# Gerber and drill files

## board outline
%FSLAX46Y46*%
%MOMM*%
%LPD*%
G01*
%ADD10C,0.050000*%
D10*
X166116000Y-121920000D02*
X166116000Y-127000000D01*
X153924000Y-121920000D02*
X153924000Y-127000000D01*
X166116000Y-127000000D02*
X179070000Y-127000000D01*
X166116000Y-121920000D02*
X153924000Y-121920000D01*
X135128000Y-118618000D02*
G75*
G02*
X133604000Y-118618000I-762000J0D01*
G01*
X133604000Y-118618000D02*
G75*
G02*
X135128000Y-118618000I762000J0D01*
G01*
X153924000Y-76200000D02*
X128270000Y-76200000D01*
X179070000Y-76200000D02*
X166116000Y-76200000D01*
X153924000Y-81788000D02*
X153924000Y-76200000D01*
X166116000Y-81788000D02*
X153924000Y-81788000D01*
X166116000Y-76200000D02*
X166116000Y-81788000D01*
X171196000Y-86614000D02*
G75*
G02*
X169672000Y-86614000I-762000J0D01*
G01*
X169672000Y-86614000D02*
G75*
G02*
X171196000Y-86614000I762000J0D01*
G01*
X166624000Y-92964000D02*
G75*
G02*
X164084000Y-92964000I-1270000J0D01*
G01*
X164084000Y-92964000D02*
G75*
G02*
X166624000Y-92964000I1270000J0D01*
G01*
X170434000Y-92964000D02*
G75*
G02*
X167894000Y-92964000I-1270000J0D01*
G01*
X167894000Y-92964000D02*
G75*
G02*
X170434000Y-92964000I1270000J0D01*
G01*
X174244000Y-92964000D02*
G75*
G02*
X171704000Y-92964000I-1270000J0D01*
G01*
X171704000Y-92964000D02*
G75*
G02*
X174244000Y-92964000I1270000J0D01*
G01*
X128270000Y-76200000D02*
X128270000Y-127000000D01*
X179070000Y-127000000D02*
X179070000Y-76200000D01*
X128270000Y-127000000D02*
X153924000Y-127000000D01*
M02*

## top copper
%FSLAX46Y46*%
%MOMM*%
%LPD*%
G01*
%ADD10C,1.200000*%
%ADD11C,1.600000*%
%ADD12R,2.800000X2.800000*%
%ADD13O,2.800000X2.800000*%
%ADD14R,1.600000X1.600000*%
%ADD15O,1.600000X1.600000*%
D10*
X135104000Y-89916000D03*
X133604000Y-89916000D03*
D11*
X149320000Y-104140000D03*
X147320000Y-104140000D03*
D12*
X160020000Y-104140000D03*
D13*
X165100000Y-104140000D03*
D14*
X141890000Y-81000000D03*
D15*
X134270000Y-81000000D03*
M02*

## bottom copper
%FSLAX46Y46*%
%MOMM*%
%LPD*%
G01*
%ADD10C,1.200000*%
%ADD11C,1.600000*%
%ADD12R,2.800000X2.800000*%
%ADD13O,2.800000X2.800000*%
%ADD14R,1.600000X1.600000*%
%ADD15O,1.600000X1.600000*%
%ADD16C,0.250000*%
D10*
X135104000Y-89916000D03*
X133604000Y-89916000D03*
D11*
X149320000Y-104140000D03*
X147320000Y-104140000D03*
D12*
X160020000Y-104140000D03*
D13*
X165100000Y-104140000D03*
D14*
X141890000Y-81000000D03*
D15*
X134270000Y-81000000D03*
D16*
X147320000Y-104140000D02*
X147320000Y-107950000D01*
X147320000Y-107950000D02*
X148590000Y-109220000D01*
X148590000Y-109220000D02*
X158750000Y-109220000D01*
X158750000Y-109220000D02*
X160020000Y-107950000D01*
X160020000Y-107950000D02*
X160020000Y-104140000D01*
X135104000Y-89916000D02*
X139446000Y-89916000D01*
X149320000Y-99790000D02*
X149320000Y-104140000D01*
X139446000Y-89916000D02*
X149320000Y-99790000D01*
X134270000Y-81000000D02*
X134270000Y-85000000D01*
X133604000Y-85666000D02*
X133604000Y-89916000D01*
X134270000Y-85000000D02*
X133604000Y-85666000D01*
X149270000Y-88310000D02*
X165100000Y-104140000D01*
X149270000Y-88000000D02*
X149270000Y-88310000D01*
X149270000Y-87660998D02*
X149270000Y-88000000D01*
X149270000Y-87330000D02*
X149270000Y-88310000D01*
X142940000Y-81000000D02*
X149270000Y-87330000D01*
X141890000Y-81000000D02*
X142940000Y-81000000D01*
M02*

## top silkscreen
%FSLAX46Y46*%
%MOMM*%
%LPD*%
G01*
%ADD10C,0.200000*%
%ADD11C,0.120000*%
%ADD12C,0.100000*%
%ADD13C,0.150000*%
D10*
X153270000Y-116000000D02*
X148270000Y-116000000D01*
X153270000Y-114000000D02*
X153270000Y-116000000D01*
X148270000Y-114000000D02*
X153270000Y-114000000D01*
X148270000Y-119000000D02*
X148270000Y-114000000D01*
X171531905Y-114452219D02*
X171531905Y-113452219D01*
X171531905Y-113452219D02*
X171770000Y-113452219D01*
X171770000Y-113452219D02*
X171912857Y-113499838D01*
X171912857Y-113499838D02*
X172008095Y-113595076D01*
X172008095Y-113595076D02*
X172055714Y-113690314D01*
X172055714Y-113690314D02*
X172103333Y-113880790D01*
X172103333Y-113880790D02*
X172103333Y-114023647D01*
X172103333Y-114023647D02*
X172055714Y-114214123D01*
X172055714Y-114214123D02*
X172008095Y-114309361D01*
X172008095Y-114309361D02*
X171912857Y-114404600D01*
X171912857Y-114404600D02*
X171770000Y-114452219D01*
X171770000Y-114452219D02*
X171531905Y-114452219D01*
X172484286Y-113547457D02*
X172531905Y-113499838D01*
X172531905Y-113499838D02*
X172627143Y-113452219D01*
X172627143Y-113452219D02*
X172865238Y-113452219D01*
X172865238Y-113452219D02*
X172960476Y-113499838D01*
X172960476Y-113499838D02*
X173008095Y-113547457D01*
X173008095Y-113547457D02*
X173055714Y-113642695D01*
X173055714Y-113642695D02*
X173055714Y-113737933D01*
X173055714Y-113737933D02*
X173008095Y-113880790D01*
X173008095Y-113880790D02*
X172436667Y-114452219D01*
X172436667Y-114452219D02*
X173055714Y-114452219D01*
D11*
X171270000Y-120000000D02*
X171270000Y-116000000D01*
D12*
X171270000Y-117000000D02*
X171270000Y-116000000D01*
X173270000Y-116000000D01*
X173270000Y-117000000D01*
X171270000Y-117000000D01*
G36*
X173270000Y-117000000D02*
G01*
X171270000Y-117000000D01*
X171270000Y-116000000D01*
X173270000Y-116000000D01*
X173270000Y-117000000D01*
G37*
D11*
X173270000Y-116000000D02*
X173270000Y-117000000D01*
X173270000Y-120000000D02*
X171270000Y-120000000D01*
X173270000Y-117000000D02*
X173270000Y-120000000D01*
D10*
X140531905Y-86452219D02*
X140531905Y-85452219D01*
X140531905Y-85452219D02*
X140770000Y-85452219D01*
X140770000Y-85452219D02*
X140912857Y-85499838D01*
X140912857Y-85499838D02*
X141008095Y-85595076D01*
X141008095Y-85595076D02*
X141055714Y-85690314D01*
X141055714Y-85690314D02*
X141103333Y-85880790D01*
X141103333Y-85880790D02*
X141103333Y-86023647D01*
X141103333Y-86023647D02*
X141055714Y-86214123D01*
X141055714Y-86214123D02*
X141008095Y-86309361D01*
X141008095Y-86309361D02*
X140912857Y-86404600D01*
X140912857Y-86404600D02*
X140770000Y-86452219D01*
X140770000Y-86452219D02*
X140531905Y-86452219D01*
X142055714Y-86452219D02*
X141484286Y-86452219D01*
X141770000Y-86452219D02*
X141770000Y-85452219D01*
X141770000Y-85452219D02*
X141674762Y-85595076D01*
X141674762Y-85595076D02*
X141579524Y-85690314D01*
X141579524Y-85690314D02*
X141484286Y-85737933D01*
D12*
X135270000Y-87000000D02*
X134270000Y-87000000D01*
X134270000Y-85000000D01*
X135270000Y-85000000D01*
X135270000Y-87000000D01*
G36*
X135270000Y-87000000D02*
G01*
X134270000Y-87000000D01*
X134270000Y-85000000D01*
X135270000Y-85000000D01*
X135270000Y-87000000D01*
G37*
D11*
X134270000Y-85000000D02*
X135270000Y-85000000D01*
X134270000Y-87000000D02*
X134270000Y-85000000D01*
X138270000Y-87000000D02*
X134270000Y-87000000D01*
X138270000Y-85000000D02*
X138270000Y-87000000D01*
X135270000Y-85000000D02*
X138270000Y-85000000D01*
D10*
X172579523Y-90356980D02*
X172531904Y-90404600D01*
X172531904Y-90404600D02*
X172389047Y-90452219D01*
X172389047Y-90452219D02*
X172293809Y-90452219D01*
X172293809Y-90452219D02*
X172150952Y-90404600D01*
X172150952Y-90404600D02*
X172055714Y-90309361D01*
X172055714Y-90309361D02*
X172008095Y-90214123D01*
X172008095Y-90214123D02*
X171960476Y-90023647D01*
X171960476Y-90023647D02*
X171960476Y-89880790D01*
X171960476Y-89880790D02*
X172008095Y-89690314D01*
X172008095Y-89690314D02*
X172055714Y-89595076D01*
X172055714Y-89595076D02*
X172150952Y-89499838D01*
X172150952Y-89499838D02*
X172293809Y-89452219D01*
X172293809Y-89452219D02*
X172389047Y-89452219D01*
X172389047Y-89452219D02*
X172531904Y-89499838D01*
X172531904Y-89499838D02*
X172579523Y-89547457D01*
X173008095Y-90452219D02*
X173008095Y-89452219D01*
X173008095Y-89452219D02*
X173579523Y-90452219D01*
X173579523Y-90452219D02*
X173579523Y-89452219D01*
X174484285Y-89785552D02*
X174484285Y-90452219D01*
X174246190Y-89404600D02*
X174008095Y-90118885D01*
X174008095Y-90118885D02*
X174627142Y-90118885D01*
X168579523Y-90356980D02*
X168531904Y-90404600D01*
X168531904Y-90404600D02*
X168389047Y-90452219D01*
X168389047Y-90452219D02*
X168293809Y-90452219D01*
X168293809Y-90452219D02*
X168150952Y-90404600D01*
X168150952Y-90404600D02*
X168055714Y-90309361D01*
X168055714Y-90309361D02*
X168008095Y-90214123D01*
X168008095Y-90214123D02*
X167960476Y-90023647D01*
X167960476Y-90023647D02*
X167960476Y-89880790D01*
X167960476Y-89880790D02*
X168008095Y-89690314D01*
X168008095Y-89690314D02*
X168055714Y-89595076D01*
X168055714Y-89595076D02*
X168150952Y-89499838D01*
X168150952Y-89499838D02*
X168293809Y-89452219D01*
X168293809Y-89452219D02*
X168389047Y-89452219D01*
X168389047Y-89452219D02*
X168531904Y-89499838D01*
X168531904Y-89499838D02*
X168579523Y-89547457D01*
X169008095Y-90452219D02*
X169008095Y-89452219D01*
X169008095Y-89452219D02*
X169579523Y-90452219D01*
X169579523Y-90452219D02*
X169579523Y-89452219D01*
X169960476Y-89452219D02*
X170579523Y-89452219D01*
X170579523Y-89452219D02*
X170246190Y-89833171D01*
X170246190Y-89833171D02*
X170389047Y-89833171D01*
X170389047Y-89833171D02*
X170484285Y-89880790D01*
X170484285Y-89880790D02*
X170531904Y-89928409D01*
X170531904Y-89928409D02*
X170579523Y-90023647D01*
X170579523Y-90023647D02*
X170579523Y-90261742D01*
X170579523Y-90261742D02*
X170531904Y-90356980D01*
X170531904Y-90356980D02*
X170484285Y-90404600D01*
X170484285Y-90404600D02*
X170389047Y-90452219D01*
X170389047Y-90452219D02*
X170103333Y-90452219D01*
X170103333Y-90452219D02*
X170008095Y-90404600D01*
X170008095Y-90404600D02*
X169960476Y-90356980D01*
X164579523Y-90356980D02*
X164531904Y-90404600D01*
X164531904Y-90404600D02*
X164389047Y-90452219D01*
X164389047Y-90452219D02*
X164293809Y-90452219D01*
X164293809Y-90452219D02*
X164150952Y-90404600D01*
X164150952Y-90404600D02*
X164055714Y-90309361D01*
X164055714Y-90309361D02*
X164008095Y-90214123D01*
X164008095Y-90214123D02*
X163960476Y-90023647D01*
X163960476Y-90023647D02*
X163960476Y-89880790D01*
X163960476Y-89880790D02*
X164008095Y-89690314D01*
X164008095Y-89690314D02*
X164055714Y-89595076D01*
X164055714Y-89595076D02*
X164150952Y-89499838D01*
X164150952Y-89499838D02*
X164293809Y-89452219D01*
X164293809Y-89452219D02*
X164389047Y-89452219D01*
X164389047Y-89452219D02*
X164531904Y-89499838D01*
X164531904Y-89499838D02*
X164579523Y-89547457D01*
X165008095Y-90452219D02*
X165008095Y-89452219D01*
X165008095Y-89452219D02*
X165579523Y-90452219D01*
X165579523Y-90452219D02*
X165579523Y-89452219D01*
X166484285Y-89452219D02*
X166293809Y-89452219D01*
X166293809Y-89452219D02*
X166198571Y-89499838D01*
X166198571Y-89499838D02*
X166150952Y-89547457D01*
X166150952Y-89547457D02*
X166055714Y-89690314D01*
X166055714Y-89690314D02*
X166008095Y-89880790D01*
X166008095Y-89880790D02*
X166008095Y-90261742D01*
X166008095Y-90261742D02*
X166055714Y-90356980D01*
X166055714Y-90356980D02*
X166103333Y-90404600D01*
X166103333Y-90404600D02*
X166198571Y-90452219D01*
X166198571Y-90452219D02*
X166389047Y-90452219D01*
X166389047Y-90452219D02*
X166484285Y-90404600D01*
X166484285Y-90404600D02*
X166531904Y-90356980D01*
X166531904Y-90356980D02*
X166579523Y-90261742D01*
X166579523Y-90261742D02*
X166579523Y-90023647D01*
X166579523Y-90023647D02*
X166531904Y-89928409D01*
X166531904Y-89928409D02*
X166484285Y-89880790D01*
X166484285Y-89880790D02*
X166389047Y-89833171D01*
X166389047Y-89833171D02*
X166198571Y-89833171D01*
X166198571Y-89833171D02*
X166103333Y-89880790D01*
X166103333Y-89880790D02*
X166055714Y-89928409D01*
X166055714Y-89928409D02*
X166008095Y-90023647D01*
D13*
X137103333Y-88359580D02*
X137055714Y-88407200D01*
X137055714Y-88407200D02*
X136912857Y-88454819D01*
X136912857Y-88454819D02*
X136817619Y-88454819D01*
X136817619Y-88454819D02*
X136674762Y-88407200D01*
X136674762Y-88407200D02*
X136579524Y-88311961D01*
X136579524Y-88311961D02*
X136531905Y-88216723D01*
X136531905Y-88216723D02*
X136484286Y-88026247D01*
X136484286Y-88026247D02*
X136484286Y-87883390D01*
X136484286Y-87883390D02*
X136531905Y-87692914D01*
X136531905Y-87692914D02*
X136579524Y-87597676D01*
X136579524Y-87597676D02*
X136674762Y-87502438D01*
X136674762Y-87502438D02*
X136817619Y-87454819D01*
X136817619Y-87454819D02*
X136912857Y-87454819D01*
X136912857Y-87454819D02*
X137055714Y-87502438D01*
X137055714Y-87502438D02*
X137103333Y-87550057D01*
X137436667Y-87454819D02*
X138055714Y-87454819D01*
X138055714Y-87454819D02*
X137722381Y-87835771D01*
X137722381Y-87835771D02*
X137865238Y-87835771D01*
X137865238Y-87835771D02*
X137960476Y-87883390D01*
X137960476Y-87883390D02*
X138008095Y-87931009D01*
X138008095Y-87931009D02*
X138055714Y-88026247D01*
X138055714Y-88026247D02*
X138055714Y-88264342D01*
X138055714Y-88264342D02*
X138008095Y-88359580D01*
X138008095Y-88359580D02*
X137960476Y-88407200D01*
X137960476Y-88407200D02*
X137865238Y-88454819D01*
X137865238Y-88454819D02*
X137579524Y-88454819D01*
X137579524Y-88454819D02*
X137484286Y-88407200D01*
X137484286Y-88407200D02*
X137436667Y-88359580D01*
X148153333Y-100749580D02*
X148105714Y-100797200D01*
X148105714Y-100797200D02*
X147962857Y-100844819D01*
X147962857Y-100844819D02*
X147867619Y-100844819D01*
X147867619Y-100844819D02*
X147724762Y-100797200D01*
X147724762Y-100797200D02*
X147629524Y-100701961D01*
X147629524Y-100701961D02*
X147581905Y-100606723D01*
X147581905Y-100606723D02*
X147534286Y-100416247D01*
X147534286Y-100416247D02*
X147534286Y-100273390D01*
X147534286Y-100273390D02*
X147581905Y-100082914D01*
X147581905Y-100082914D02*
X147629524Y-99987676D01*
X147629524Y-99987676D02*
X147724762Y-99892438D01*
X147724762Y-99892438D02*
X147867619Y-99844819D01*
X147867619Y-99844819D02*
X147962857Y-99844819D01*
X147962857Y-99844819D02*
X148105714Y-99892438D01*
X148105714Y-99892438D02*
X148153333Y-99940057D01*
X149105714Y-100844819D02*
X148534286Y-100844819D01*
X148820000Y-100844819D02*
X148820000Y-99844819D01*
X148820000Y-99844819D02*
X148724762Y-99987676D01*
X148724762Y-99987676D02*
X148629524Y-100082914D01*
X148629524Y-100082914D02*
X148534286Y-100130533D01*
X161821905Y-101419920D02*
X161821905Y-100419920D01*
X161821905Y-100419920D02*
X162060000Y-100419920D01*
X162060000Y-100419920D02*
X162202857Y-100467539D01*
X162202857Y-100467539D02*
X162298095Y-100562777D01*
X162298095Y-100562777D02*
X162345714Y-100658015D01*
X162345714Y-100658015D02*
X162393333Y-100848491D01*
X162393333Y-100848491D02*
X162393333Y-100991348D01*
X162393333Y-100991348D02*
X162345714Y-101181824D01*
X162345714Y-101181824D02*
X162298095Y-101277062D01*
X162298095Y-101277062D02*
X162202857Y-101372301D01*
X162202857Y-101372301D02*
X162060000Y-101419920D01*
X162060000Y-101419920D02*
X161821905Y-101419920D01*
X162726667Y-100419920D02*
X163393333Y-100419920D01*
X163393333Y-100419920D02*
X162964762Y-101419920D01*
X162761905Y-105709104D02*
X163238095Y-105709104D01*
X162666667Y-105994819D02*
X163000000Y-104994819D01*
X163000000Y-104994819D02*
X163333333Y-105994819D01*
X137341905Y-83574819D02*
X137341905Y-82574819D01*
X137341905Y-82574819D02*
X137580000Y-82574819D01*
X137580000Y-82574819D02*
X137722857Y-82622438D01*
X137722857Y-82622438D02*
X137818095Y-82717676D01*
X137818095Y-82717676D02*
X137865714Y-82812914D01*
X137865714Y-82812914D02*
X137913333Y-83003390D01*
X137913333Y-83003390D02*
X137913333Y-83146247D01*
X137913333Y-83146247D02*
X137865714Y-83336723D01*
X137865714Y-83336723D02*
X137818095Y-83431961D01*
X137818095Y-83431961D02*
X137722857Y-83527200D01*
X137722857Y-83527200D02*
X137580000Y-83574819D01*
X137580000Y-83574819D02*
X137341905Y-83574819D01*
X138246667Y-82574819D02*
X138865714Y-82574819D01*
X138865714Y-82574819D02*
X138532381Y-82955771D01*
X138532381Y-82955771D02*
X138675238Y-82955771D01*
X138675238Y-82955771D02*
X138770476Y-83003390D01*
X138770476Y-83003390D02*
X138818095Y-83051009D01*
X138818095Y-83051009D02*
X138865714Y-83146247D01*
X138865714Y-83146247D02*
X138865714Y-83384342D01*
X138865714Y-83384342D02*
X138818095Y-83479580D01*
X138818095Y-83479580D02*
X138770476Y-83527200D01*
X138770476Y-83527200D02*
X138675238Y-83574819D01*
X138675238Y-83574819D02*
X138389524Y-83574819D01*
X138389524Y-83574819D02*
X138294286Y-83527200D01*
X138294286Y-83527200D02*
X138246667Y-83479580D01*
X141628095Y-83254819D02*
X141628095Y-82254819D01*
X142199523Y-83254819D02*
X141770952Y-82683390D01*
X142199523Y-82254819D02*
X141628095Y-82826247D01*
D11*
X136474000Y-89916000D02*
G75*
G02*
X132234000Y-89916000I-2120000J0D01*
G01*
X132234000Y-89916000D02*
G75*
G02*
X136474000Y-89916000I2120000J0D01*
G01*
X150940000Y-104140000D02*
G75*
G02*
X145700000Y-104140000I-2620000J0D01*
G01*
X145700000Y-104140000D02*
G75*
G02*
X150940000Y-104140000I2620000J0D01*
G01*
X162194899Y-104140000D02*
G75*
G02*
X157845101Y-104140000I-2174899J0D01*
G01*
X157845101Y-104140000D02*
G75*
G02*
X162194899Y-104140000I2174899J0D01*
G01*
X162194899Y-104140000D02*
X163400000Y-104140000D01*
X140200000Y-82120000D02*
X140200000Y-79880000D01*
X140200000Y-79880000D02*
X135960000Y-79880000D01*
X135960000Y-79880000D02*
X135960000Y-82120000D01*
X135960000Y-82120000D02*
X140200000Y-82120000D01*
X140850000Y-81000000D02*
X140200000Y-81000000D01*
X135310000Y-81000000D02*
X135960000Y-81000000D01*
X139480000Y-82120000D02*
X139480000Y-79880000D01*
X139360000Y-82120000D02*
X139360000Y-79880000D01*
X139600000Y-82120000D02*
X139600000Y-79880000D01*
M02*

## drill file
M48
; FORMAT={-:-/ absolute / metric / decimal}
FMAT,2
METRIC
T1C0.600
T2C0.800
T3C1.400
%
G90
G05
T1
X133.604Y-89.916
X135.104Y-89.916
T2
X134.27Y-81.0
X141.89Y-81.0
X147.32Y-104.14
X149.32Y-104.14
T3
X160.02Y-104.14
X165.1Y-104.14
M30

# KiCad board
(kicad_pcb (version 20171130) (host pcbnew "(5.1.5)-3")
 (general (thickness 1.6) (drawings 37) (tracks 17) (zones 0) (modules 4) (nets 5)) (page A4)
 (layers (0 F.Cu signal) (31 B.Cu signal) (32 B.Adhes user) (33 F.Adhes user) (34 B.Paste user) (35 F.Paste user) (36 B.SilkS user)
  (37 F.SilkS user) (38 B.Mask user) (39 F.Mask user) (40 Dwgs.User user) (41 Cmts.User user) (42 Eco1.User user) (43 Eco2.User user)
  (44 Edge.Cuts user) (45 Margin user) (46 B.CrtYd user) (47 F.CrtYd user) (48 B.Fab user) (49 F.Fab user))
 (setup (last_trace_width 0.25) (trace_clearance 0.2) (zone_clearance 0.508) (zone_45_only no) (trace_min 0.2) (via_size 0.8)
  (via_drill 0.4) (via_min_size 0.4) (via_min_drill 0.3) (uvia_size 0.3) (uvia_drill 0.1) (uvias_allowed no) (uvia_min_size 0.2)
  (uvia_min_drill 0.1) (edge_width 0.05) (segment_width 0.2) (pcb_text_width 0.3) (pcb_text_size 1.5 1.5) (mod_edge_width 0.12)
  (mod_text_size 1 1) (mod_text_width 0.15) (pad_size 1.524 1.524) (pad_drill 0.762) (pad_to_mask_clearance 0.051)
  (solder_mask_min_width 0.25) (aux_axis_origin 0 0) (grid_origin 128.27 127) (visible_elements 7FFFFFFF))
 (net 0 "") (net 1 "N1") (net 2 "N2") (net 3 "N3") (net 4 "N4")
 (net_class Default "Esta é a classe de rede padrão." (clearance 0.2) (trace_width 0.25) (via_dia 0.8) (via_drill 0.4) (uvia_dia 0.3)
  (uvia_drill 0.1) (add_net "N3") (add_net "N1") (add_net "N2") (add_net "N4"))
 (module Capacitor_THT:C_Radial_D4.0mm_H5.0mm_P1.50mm (layer F.Cu) (at 133.604 89.916)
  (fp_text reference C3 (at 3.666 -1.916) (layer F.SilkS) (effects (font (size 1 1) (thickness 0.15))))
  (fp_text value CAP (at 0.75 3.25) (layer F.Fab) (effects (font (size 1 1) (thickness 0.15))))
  (fp_circle (center 0.75 0) (end 2.87 0) (layer F.SilkS) (width 0.12))
  (pad 2 thru_hole circle (at 1.5 0) (size 1.2 1.2) (drill 0.6) (layers *.Cu *.Mask) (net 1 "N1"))
  (pad 1 thru_hole circle (at 0 0) (size 1.2 1.2) (drill 0.6) (layers *.Cu *.Mask) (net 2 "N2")))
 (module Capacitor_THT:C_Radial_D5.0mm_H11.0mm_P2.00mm (layer F.Cu) (at 147.32 104.14)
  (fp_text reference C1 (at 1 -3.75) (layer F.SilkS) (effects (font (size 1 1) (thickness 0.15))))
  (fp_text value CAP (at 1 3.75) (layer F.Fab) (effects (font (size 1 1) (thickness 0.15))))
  (fp_circle (center 1 0) (end 3.62 0) (layer F.SilkS) (width 0.12))
  (pad 2 thru_hole circle (at 2 0) (size 1.6 1.6) (drill 0.8) (layers *.Cu *.Mask) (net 1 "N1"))
  (pad 1 thru_hole circle (at 0 0) (size 1.6 1.6) (drill 0.8) (layers *.Cu *.Mask) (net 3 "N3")))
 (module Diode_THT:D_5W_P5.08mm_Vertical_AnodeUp (layer F.Cu) (at 160.02 104.14)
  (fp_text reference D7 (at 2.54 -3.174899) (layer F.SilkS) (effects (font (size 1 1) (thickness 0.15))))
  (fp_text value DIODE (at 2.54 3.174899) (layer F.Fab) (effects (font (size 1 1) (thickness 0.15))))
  (fp_circle (center 0 0) (end 2.174899 0) (layer F.SilkS) (width 0.12))
  (fp_line (start 2.174899 0) (end 3.38 0) (layer F.SilkS) (width 0.12))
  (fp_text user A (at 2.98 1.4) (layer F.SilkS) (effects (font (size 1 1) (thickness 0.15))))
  (pad 1 thru_hole rect (at 0 0) (size 2.8 2.8) (drill 1.4) (layers *.Cu *.Mask) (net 3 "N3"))
  (pad 2 thru_hole oval (at 5.08 0) (size 2.8 2.8) (drill 1.4) (layers *.Cu *.Mask) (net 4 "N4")))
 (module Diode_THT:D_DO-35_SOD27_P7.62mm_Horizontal (layer F.Cu) (at 141.89 81 180)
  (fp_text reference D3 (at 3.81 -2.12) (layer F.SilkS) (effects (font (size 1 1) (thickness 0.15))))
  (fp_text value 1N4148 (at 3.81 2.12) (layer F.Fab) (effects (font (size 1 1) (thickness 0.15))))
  (fp_line (start 1.69 -1.12) (end 1.69 1.12) (layer F.SilkS) (width 0.12))
  (fp_line (start 1.69 1.12) (end 5.93 1.12) (layer F.SilkS) (width 0.12))
  (fp_line (start 5.93 1.12) (end 5.93 -1.12) (layer F.SilkS) (width 0.12))
  (fp_line (start 5.93 -1.12) (end 1.69 -1.12) (layer F.SilkS) (width 0.12))
  (fp_line (start 1.04 0) (end 1.69 0) (layer F.SilkS) (width 0.12))
  (fp_line (start 6.58 0) (end 5.93 0) (layer F.SilkS) (width 0.12))
  (fp_line (start 2.41 -1.12) (end 2.41 1.12) (layer F.SilkS) (width 0.12))
  (fp_line (start 2.53 -1.12) (end 2.53 1.12) (layer F.SilkS) (width 0.12))
  (fp_line (start 2.29 -1.12) (end 2.29 1.12) (layer F.SilkS) (width 0.12))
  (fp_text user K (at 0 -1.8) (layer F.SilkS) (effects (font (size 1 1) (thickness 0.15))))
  (pad 1 thru_hole rect (at 0 0 180) (size 1.6 1.6) (drill 0.8) (layers *.Cu *.Mask) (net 4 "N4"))
  (pad 2 thru_hole oval (at 7.62 0 180) (size 1.6 1.6) (drill 0.8) (layers *.Cu *.Mask) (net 2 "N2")))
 (gr_line (start 153.27 116) (end 148.27 116) (layer F.SilkS) (width 0.2))
 (gr_line (start 153.27 114) (end 153.27 116) (layer F.SilkS) (width 0.2))
 (gr_line (start 148.27 114) (end 153.27 114) (layer F.SilkS) (width 0.2))
 (gr_line (start 148.27 119) (end 148.27 114) (layer F.SilkS) (width 0.2))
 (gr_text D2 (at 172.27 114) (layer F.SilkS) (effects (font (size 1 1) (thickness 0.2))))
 (gr_line (start 171.27 120) (end 171.27 116) (layer F.SilkS) (width 0.12))
 (gr_poly (pts (xy 171.27 117) (xy 171.27 116) (xy 173.27 116) (xy 173.27 117)) (layer F.SilkS) (width 0.1))
 (gr_line (start 173.27 116) (end 173.27 117) (layer F.SilkS) (width 0.12))
 (gr_line (start 173.27 120) (end 171.27 120) (layer F.SilkS) (width 0.12))
 (gr_line (start 173.27 117) (end 173.27 120) (layer F.SilkS) (width 0.12))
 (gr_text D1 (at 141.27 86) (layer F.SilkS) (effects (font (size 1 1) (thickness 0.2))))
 (gr_poly (pts (xy 135.27 87) (xy 134.27 87) (xy 134.27 85) (xy 135.27 85)) (layer F.SilkS) (width 0.1))
 (gr_line (start 134.27 85) (end 135.27 85) (layer F.SilkS) (width 0.12))
 (gr_line (start 134.27 87) (end 134.27 85) (layer F.SilkS) (width 0.12))
 (gr_line (start 138.27 87) (end 134.27 87) (layer F.SilkS) (width 0.12))
 (gr_line (start 138.27 85) (end 138.27 87) (layer F.SilkS) (width 0.12))
 (gr_line (start 135.27 85) (end 138.27 85) (layer F.SilkS) (width 0.12))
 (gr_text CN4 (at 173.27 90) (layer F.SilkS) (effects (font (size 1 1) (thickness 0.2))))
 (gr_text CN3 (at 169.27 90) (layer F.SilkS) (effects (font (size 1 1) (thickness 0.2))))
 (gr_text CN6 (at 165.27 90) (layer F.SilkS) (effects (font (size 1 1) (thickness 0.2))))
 (gr_line (start 166.116 121.92) (end 166.116 127) (layer Edge.Cuts) (width 0.05))
 (gr_line (start 153.924 121.92) (end 153.924 127) (layer Edge.Cuts) (width 0.05))
 (gr_line (start 166.116 127) (end 179.07 127) (layer Edge.Cuts) (width 0.05))
 (gr_line (start 166.116 121.92) (end 153.924 121.92) (layer Edge.Cuts) (width 0.05))
 (gr_circle (center 134.366 118.618) (end 135.128 118.618) (layer Edge.Cuts) (width 0.05))
 (gr_line (start 153.924 76.2) (end 128.27 76.2) (layer Edge.Cuts) (width 0.05))
 (gr_line (start 179.07 76.2) (end 166.116 76.2) (layer Edge.Cuts) (width 0.05))
 (gr_line (start 153.924 81.788) (end 153.924 76.2) (layer Edge.Cuts) (width 0.05))
 (gr_line (start 166.116 81.788) (end 153.924 81.788) (layer Edge.Cuts) (width 0.05))
 (gr_line (start 166.116 76.2) (end 166.116 81.788) (layer Edge.Cuts) (width 0.05))
 (gr_circle (center 170.434 86.614) (end 171.196 86.614) (layer Edge.Cuts) (width 0.05))
 (gr_circle (center 165.354 92.964) (end 166.624 92.964) (layer Edge.Cuts) (width 0.05))
 (gr_circle (center 169.164 92.964) (end 170.434 92.964) (layer Edge.Cuts) (width 0.05))
 (gr_circle (center 172.974 92.964) (end 174.244 92.964) (layer Edge.Cuts) (width 0.05))
 (gr_line (start 128.27 76.2) (end 128.27 127) (layer Edge.Cuts) (width 0.05))
 (gr_line (start 179.07 127) (end 179.07 76.2) (layer Edge.Cuts) (width 0.05))
 (gr_line (start 128.27 127) (end 153.924 127) (layer Edge.Cuts) (width 0.05))
 (segment (start 147.32 104.14) (end 147.32 107.95) (width 0.25) (layer B.Cu) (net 3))
 (segment (start 147.32 107.95) (end 148.59 109.22) (width 0.25) (layer B.Cu) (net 3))
 (segment (start 148.59 109.22) (end 158.75 109.22) (width 0.25) (layer B.Cu) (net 3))
 (segment (start 158.75 109.22) (end 160.02 107.95) (width 0.25) (layer B.Cu) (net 3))
 (segment (start 160.02 107.95) (end 160.02 104.14) (width 0.25) (layer B.Cu) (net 3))
 (segment (start 135.104 89.916) (end 139.446 89.916) (width 0.25) (layer B.Cu) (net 1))
 (segment (start 149.32 99.79) (end 149.32 104.14) (width 0.25) (layer B.Cu) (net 1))
 (segment (start 139.446 89.916) (end 149.32 99.79) (width 0.25) (layer B.Cu) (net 1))
 (segment (start 134.27 81) (end 134.27 85) (width 0.25) (layer B.Cu) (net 2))
 (segment (start 133.604 85.666) (end 133.604 89.916) (width 0.25) (layer B.Cu) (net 2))
 (segment (start 134.27 85) (end 133.604 85.666) (width 0.25) (layer B.Cu) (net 2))
 (segment (start 149.27 88.31) (end 165.1 104.14) (width 0.25) (layer B.Cu) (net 4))
 (segment (start 149.27 88) (end 149.27 88.31) (width 0.25) (layer B.Cu) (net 4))
 (segment (start 149.27 87.660998) (end 149.27 88) (width 0.25) (layer B.Cu) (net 4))
 (segment (start 149.27 87.33) (end 149.27 88.31) (width 0.25) (layer B.Cu) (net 4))
 (segment (start 142.94 81) (end 149.27 87.33) (width 0.25) (layer B.Cu) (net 4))
 (segment (start 141.89 81) (end 142.94 81) (width 0.25) (layer B.Cu) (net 4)))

